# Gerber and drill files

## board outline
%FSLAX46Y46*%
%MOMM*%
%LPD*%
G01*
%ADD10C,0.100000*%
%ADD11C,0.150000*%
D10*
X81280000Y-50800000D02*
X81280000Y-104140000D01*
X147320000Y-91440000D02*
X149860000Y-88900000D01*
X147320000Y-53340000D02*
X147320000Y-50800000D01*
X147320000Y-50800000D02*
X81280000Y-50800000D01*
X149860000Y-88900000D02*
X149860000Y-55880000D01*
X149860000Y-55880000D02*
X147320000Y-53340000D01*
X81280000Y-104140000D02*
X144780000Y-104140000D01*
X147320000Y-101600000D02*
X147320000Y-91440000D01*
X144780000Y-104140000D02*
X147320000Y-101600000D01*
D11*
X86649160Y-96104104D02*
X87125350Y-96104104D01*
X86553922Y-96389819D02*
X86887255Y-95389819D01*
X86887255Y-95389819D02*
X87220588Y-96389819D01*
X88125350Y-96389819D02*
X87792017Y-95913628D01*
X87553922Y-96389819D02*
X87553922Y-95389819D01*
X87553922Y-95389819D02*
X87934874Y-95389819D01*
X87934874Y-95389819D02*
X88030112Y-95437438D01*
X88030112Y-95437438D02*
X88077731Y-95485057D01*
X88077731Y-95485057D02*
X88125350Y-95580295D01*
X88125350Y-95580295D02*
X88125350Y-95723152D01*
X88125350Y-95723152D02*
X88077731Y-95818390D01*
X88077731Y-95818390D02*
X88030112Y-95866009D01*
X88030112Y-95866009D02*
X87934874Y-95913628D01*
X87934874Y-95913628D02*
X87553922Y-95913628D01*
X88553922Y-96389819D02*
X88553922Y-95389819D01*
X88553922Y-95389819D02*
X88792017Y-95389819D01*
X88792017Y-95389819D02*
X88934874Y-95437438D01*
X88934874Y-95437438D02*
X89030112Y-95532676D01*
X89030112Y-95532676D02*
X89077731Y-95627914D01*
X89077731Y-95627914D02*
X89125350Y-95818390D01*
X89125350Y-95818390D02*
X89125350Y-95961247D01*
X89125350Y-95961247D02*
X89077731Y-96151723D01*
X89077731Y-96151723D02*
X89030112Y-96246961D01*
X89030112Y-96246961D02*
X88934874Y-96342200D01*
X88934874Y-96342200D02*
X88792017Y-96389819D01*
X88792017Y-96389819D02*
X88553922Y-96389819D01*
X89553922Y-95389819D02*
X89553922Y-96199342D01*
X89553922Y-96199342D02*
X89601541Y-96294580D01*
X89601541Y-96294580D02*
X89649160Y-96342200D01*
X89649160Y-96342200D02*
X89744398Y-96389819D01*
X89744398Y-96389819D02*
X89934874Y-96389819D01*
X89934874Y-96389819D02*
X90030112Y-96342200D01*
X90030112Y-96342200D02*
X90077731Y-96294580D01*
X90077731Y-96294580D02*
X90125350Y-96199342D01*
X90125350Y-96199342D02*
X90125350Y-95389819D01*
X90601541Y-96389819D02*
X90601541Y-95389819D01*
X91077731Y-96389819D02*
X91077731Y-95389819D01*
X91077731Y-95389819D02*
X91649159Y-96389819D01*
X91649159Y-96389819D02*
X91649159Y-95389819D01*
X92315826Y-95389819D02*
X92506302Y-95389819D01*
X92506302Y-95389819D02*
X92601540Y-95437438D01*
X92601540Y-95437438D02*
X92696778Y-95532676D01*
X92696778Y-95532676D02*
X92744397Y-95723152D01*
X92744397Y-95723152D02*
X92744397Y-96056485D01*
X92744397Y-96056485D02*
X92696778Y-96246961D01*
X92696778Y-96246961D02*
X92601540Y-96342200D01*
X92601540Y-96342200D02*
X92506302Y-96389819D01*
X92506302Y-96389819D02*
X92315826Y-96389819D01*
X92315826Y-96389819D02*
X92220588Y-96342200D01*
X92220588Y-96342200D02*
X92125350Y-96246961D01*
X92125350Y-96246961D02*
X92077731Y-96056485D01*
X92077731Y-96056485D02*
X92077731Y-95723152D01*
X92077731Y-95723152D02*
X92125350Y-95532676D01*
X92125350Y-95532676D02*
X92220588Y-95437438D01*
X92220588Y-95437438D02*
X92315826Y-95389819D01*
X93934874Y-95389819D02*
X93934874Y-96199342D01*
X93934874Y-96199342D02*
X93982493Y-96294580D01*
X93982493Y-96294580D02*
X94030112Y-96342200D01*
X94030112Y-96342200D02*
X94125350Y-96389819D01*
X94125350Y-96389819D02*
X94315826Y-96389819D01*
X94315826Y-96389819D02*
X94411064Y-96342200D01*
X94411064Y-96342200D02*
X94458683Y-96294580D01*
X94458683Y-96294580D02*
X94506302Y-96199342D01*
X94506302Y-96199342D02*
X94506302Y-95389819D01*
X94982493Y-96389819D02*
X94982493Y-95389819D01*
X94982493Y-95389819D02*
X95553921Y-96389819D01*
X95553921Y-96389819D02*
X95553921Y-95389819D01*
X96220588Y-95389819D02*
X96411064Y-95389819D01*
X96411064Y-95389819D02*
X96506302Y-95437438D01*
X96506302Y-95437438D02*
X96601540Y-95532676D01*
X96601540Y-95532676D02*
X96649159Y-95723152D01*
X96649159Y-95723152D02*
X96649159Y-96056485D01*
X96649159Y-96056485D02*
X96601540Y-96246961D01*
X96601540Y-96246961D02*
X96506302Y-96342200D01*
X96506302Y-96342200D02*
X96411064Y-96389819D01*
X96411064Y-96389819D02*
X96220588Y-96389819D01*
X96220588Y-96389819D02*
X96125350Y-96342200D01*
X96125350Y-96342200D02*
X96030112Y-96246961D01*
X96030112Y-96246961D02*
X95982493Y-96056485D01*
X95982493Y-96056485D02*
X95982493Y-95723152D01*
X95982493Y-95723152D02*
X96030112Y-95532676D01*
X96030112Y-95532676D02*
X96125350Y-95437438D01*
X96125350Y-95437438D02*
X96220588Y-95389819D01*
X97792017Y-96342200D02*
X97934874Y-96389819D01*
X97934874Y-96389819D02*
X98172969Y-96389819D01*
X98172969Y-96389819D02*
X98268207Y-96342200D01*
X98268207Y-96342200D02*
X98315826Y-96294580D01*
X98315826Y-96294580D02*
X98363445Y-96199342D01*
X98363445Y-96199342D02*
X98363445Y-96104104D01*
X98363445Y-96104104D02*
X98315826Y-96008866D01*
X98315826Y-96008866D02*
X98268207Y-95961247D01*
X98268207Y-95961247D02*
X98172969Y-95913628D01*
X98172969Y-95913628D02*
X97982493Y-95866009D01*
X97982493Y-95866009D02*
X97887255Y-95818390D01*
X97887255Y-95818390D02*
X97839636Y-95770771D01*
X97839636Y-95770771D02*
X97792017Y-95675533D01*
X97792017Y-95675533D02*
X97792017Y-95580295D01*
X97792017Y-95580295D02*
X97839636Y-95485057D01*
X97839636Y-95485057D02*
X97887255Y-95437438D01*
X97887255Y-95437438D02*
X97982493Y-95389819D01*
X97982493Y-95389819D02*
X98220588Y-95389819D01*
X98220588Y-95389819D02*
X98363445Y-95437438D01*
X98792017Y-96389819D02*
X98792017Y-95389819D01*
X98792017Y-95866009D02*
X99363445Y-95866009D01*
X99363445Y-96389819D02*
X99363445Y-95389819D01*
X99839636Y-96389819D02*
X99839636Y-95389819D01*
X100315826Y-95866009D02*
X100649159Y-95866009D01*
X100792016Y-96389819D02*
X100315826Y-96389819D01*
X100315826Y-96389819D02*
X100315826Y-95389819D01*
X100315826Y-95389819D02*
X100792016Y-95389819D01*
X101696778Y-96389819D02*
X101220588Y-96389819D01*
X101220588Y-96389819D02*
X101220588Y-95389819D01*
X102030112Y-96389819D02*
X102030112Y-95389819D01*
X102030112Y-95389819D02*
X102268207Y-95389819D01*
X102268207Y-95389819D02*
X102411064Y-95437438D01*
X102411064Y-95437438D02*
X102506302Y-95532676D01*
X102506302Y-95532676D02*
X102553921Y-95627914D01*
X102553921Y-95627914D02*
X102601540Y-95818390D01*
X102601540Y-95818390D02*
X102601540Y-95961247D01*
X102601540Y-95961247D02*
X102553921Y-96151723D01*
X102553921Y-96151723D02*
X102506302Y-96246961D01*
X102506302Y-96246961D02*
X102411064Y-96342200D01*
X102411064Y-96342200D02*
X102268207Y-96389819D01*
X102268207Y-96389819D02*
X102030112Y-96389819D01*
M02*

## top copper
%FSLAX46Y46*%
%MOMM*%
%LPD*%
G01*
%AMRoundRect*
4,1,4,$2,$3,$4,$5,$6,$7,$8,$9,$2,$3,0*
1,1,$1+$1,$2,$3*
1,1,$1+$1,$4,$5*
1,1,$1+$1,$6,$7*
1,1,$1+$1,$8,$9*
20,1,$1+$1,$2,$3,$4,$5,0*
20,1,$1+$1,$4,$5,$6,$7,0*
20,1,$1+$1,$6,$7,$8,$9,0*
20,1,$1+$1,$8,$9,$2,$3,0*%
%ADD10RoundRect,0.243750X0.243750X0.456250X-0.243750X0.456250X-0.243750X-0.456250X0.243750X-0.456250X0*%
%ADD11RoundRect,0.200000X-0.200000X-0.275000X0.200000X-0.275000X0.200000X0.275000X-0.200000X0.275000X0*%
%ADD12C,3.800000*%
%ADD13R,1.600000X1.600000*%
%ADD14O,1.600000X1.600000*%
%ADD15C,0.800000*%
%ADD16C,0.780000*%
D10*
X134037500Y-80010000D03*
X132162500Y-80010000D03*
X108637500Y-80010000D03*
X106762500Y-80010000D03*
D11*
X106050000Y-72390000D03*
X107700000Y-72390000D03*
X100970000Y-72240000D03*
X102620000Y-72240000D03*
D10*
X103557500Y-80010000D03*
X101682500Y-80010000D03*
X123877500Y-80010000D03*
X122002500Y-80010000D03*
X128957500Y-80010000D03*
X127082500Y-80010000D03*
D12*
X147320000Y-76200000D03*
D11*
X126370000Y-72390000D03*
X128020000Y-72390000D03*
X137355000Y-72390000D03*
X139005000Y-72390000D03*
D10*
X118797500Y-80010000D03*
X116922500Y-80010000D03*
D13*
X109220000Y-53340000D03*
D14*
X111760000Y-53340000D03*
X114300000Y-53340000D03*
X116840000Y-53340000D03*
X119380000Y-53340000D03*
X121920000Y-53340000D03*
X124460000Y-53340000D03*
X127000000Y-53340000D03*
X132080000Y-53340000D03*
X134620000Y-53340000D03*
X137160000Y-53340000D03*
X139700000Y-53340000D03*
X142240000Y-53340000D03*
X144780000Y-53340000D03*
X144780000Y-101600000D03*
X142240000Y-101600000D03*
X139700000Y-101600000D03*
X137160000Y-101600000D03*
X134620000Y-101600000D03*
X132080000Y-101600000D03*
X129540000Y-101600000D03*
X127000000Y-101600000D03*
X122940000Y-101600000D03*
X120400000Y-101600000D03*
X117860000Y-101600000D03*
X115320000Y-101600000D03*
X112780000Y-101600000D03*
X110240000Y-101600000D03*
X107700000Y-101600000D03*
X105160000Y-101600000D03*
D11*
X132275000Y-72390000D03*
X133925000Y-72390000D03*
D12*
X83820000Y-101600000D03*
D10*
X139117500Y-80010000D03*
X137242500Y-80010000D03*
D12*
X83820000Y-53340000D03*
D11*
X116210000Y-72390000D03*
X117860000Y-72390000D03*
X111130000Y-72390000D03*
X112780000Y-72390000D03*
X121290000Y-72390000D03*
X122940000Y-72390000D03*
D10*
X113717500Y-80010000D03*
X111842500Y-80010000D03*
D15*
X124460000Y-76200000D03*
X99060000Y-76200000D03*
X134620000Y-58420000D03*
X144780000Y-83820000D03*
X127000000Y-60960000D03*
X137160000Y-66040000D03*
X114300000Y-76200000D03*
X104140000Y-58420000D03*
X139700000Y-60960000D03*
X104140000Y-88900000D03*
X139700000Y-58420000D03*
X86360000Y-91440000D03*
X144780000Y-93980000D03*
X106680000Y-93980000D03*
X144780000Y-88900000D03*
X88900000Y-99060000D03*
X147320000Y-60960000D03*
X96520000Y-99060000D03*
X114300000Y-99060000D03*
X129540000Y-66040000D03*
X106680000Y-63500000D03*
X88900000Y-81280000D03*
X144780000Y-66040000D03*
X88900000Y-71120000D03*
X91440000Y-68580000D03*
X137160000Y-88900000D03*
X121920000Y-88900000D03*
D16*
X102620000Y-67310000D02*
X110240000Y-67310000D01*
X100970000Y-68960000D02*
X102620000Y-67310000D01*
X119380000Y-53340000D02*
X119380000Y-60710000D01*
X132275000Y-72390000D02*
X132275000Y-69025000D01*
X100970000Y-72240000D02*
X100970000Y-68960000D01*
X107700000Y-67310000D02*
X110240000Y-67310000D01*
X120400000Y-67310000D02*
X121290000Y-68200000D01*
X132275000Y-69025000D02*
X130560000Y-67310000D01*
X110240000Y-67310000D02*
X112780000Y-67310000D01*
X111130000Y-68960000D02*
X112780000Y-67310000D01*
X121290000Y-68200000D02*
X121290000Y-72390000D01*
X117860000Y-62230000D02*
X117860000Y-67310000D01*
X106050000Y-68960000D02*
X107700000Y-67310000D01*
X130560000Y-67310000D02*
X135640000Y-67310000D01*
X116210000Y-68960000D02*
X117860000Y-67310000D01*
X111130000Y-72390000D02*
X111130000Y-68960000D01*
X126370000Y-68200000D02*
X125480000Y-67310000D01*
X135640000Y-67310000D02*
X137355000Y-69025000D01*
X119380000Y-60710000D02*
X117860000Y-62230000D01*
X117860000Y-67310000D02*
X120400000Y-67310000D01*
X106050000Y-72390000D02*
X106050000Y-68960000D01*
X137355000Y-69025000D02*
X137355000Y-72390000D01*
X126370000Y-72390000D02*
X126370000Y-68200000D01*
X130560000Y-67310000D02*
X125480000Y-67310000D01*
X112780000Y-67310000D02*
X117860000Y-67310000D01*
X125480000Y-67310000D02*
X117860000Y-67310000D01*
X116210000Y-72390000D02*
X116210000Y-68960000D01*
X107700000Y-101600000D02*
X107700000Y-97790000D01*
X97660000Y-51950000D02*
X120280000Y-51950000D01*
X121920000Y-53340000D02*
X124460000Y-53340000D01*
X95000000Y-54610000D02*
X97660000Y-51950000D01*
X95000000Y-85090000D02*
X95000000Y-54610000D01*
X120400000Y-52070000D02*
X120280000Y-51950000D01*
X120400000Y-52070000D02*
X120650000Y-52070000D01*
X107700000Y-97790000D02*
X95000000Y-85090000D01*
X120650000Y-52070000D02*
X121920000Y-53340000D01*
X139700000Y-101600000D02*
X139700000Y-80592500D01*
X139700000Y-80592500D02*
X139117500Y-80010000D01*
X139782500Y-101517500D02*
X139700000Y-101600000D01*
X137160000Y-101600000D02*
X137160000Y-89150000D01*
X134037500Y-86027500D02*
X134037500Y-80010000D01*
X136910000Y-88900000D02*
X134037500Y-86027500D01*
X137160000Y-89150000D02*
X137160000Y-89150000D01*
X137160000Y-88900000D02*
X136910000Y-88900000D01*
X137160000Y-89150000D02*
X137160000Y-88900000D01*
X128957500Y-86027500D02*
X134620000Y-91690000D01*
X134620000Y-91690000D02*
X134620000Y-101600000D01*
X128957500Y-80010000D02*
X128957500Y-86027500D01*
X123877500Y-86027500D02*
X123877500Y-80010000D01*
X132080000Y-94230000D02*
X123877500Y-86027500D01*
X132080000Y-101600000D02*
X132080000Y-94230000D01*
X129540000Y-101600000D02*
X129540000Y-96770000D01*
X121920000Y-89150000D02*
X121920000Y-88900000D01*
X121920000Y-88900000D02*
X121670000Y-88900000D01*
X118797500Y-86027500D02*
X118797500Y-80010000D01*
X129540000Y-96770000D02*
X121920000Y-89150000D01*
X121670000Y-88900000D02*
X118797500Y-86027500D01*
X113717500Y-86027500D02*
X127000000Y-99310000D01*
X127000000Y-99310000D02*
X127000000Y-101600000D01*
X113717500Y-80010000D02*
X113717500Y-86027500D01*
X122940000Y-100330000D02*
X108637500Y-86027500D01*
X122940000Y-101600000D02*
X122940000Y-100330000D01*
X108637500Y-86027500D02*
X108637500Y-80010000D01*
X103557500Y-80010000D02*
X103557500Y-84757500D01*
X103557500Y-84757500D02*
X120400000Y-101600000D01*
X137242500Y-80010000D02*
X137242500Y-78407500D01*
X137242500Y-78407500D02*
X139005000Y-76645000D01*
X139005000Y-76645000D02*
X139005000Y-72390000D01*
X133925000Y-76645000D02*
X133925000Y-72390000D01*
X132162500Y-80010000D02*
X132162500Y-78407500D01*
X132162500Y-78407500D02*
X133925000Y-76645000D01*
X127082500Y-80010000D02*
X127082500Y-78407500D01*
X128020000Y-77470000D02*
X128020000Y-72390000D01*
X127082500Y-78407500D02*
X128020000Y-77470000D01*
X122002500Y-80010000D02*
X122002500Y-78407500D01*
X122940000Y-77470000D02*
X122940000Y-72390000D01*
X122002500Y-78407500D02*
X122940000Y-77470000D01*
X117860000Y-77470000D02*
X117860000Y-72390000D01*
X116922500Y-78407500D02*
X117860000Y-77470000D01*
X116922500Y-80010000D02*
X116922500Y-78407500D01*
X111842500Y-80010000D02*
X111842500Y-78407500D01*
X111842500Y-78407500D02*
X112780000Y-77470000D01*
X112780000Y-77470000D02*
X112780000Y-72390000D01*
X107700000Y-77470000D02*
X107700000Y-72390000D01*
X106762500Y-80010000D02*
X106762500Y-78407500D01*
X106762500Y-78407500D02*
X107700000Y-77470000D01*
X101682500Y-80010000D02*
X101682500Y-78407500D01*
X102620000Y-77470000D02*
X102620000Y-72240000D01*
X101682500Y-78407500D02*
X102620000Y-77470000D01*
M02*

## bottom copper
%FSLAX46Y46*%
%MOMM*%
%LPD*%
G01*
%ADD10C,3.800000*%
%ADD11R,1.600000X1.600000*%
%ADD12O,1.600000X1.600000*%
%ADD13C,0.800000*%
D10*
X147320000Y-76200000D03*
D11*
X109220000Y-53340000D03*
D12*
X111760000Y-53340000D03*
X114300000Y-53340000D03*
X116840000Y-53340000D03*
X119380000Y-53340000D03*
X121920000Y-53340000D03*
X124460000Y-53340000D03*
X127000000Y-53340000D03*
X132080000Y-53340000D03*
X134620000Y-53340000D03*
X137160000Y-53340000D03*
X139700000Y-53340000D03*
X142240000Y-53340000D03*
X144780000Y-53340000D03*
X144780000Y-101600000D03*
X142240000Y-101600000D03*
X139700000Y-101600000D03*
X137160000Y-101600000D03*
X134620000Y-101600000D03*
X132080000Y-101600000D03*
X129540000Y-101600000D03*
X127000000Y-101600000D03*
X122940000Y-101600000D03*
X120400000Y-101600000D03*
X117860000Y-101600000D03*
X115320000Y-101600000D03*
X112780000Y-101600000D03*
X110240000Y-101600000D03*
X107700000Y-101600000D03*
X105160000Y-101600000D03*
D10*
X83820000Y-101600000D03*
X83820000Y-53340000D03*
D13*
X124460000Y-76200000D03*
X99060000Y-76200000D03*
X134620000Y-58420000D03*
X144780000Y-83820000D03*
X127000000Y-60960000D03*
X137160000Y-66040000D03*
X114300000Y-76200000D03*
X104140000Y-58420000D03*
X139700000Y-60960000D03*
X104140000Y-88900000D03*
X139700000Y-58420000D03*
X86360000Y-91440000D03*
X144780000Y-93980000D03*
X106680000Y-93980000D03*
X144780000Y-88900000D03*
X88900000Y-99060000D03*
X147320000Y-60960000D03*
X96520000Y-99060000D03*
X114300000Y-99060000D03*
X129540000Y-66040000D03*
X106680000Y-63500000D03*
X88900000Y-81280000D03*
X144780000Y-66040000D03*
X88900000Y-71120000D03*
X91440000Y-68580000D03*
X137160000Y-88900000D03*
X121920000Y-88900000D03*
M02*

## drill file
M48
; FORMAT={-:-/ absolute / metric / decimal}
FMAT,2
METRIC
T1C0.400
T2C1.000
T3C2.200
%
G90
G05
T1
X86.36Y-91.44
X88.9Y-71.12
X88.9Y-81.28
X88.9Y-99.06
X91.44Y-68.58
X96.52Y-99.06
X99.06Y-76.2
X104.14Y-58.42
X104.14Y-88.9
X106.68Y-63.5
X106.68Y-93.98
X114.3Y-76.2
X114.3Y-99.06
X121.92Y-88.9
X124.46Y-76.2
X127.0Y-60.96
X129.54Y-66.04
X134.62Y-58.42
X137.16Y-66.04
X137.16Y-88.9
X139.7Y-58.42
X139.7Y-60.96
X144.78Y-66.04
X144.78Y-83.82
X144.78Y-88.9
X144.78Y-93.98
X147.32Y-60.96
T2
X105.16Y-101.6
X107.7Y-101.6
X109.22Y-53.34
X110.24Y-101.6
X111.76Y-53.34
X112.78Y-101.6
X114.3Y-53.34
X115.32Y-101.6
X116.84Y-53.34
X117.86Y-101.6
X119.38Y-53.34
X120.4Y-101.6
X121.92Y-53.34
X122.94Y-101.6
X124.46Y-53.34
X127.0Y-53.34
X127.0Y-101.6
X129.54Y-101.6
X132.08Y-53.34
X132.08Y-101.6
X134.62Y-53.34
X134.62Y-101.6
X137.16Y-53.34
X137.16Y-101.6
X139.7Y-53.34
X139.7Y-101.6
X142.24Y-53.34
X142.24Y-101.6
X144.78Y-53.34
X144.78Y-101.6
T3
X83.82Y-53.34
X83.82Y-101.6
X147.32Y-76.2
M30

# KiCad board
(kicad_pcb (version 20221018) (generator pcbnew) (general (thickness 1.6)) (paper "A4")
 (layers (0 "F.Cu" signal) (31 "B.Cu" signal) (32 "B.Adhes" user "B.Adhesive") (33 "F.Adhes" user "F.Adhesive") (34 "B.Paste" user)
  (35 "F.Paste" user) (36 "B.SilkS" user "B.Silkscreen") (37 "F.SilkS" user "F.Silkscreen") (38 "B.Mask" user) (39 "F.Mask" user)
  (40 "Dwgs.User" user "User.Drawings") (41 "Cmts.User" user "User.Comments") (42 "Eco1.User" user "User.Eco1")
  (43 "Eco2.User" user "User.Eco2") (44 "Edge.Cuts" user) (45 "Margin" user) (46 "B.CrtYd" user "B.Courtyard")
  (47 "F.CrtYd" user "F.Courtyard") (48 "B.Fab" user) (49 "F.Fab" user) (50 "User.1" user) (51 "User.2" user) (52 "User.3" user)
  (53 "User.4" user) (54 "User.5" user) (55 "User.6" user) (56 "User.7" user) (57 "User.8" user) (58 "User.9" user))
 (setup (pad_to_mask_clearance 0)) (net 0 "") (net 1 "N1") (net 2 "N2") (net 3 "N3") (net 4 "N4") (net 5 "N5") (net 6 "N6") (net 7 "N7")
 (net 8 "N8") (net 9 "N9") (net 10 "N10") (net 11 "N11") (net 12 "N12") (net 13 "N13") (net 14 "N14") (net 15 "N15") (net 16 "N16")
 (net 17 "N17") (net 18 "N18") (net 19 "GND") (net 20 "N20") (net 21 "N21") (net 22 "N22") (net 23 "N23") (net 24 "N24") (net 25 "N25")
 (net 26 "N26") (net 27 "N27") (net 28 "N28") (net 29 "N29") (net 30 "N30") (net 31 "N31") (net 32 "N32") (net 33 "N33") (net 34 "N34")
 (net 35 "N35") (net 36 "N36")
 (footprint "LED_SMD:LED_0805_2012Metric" (layer "F.Cu") (at 133.1 80.01 180)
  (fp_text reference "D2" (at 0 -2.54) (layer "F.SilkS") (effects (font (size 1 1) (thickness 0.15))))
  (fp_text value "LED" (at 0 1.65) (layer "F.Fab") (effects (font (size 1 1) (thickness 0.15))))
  (pad "1" smd roundrect (at -0.9375 0 180) (size 0.975 1.4) (layers "F.Cu" "F.Paste" "F.Mask") (roundrect_rratio 0.25) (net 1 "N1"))
  (pad "2" smd roundrect (at 0.9375 0 180) (size 0.975 1.4) (layers "F.Cu" "F.Paste" "F.Mask") (roundrect_rratio 0.25) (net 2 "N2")))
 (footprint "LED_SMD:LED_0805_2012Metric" (layer "F.Cu") (at 107.7 80.01 180)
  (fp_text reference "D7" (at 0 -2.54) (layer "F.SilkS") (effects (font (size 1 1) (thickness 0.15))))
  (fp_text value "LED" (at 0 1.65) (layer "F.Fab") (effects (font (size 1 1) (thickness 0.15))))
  (pad "1" smd roundrect (at -0.9375 0 180) (size 0.975 1.4) (layers "F.Cu" "F.Paste" "F.Mask") (roundrect_rratio 0.25) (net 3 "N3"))
  (pad "2" smd roundrect (at 0.9375 0 180) (size 0.975 1.4) (layers "F.Cu" "F.Paste" "F.Mask") (roundrect_rratio 0.25) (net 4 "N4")))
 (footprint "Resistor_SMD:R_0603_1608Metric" (layer "F.Cu") (at 106.875 72.39)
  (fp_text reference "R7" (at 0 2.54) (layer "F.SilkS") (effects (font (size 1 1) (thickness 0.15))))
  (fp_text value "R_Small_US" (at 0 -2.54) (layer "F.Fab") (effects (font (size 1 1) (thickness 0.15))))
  (pad "1" smd roundrect (at -0.825 0) (size 0.8 0.95) (layers "F.Cu" "F.Paste" "F.Mask") (roundrect_rratio 0.25) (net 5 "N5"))
  (pad "2" smd roundrect (at 0.825 0) (size 0.8 0.95) (layers "F.Cu" "F.Paste" "F.Mask") (roundrect_rratio 0.25) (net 4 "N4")))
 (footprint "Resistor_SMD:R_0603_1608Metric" (layer "F.Cu") (at 101.795 72.24)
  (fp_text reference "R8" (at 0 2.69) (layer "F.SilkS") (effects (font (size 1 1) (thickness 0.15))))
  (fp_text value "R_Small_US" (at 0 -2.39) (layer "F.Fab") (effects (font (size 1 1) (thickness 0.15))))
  (pad "1" smd roundrect (at -0.825 0) (size 0.8 0.95) (layers "F.Cu" "F.Paste" "F.Mask") (roundrect_rratio 0.25) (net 5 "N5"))
  (pad "2" smd roundrect (at 0.825 0) (size 0.8 0.95) (layers "F.Cu" "F.Paste" "F.Mask") (roundrect_rratio 0.25) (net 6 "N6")))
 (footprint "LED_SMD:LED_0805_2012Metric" (layer "F.Cu") (at 102.62 80.01 180)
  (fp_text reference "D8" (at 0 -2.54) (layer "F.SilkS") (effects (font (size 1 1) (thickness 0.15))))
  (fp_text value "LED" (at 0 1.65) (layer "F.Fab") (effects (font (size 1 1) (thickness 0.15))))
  (pad "1" smd roundrect (at -0.9375 0 180) (size 0.975 1.4) (layers "F.Cu" "F.Paste" "F.Mask") (roundrect_rratio 0.25) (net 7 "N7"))
  (pad "2" smd roundrect (at 0.9375 0 180) (size 0.975 1.4) (layers "F.Cu" "F.Paste" "F.Mask") (roundrect_rratio 0.25) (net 6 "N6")))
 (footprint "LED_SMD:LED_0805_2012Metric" (layer "F.Cu") (at 122.94 80.01 180)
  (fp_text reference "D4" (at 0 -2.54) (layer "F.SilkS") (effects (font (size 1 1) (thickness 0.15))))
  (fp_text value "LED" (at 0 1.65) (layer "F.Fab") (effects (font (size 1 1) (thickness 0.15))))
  (pad "1" smd roundrect (at -0.9375 0 180) (size 0.975 1.4) (layers "F.Cu" "F.Paste" "F.Mask") (roundrect_rratio 0.25) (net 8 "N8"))
  (pad "2" smd roundrect (at 0.9375 0 180) (size 0.975 1.4) (layers "F.Cu" "F.Paste" "F.Mask") (roundrect_rratio 0.25) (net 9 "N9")))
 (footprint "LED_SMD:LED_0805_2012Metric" (layer "F.Cu") (at 128.02 80.01 180)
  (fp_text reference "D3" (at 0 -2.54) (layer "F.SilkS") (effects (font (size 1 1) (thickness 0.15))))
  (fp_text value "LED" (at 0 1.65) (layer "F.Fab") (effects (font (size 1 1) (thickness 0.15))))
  (pad "1" smd roundrect (at -0.9375 0 180) (size 0.975 1.4) (layers "F.Cu" "F.Paste" "F.Mask") (roundrect_rratio 0.25) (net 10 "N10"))
  (pad "2" smd roundrect (at 0.9375 0 180) (size 0.975 1.4) (layers "F.Cu" "F.Paste" "F.Mask") (roundrect_rratio 0.25) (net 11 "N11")))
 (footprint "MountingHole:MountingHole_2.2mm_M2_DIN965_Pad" (layer "F.Cu") (at 147.32 76.2)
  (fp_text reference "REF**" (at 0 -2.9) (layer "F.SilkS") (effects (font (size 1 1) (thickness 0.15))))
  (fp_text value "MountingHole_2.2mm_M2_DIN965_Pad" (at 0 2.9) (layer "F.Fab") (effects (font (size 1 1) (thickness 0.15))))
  (pad "1" thru_hole circle (at 0 0) (size 3.8 3.8) (drill 2.2) (layers "*.Cu" "*.Mask")))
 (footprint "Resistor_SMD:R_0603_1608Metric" (layer "F.Cu") (at 127.195 72.39)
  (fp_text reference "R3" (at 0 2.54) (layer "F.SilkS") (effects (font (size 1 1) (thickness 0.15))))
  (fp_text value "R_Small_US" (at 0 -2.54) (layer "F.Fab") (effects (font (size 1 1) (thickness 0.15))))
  (pad "1" smd roundrect (at -0.825 0) (size 0.8 0.95) (layers "F.Cu" "F.Paste" "F.Mask") (roundrect_rratio 0.25) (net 5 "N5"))
  (pad "2" smd roundrect (at 0.825 0) (size 0.8 0.95) (layers "F.Cu" "F.Paste" "F.Mask") (roundrect_rratio 0.25) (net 11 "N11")))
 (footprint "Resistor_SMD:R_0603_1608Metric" (layer "F.Cu") (at 138.18 72.39)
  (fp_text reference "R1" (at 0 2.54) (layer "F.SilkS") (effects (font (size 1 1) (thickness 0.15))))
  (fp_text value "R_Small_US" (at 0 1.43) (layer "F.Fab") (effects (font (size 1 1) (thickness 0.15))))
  (pad "1" smd roundrect (at -0.825 0) (size 0.8 0.95) (layers "F.Cu" "F.Paste" "F.Mask") (roundrect_rratio 0.25) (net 5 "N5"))
  (pad "2" smd roundrect (at 0.825 0) (size 0.8 0.95) (layers "F.Cu" "F.Paste" "F.Mask") (roundrect_rratio 0.25) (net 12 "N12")))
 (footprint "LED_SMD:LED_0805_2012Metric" (layer "F.Cu") (at 117.86 80.01 180)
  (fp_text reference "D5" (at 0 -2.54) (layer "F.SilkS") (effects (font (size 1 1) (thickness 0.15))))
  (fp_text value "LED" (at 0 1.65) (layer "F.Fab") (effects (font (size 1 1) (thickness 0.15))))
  (pad "1" smd roundrect (at -0.9375 0 180) (size 0.975 1.4) (layers "F.Cu" "F.Paste" "F.Mask") (roundrect_rratio 0.25) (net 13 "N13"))
  (pad "2" smd roundrect (at 0.9375 0 180) (size 0.975 1.4) (layers "F.Cu" "F.Paste" "F.Mask") (roundrect_rratio 0.25) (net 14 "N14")))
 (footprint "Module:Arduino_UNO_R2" (layer "F.Cu") (at 109.22 53.34)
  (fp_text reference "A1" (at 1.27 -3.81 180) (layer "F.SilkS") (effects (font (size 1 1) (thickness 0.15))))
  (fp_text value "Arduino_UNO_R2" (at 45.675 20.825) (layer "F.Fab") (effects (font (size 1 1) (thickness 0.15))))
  (pad "1" thru_hole rect (at 0 0 90) (size 1.6 1.6) (drill 1) (layers "*.Cu" "*.Mask") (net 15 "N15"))
  (pad "2" thru_hole oval (at 2.54 0 90) (size 1.6 1.6) (drill 1) (layers "*.Cu" "*.Mask") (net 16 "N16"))
  (pad "3" thru_hole oval (at 5.08 0 90) (size 1.6 1.6) (drill 1) (layers "*.Cu" "*.Mask") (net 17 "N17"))
  (pad "4" thru_hole oval (at 7.62 0 90) (size 1.6 1.6) (drill 1) (layers "*.Cu" "*.Mask") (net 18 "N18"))
  (pad "5" thru_hole oval (at 10.16 0 90) (size 1.6 1.6) (drill 1) (layers "*.Cu" "*.Mask") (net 5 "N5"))
  (pad "6" thru_hole oval (at 12.7 0 90) (size 1.6 1.6) (drill 1) (layers "*.Cu" "*.Mask") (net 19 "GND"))
  (pad "7" thru_hole oval (at 15.24 0 90) (size 1.6 1.6) (drill 1) (layers "*.Cu" "*.Mask") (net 19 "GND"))
  (pad "8" thru_hole oval (at 17.78 0 90) (size 1.6 1.6) (drill 1) (layers "*.Cu" "*.Mask") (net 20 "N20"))
  (pad "9" thru_hole oval (at 22.86 0 90) (size 1.6 1.6) (drill 1) (layers "*.Cu" "*.Mask") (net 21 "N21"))
  (pad "10" thru_hole oval (at 25.4 0 90) (size 1.6 1.6) (drill 1) (layers "*.Cu" "*.Mask") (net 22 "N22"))
  (pad "11" thru_hole oval (at 27.94 0 90) (size 1.6 1.6) (drill 1) (layers "*.Cu" "*.Mask") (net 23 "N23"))
  (pad "12" thru_hole oval (at 30.48 0 90) (size 1.6 1.6) (drill 1) (layers "*.Cu" "*.Mask") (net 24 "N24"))
  (pad "13" thru_hole oval (at 33.02 0 90) (size 1.6 1.6) (drill 1) (layers "*.Cu" "*.Mask") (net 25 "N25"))
  (pad "14" thru_hole oval (at 35.56 0 90) (size 1.6 1.6) (drill 1) (layers "*.Cu" "*.Mask") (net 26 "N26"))
  (pad "15" thru_hole oval (at 35.56 48.26 90) (size 1.6 1.6) (drill 1) (layers "*.Cu" "*.Mask") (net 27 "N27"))
  (pad "16" thru_hole oval (at 33.02 48.26 90) (size 1.6 1.6) (drill 1) (layers "*.Cu" "*.Mask") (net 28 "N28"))
  (pad "17" thru_hole oval (at 30.48 48.26 90) (size 1.6 1.6) (drill 1) (layers "*.Cu" "*.Mask") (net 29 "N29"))
  (pad "18" thru_hole oval (at 27.94 48.26 90) (size 1.6 1.6) (drill 1) (layers "*.Cu" "*.Mask") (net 1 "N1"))
  (pad "19" thru_hole oval (at 25.4 48.26 90) (size 1.6 1.6) (drill 1) (layers "*.Cu" "*.Mask") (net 10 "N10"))
  (pad "20" thru_hole oval (at 22.86 48.26 90) (size 1.6 1.6) (drill 1) (layers "*.Cu" "*.Mask") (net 8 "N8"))
  (pad "21" thru_hole oval (at 20.32 48.26 90) (size 1.6 1.6) (drill 1) (layers "*.Cu" "*.Mask") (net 13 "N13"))
  (pad "22" thru_hole oval (at 17.78 48.26 90) (size 1.6 1.6) (drill 1) (layers "*.Cu" "*.Mask") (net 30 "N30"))
  (pad "23" thru_hole oval (at 13.72 48.26 90) (size 1.6 1.6) (drill 1) (layers "*.Cu" "*.Mask") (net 3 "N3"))
  (pad "24" thru_hole oval (at 11.18 48.26 90) (size 1.6 1.6) (drill 1) (layers "*.Cu" "*.Mask") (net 7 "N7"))
  (pad "25" thru_hole oval (at 8.64 48.26 90) (size 1.6 1.6) (drill 1) (layers "*.Cu" "*.Mask") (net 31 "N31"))
  (pad "26" thru_hole oval (at 6.1 48.26 90) (size 1.6 1.6) (drill 1) (layers "*.Cu" "*.Mask") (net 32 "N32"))
  (pad "27" thru_hole oval (at 3.56 48.26 90) (size 1.6 1.6) (drill 1) (layers "*.Cu" "*.Mask") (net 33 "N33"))
  (pad "28" thru_hole oval (at 1.02 48.26 90) (size 1.6 1.6) (drill 1) (layers "*.Cu" "*.Mask") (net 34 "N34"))
  (pad "29" thru_hole oval (at -1.52 48.26 90) (size 1.6 1.6) (drill 1) (layers "*.Cu" "*.Mask") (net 19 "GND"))
  (pad "30" thru_hole oval (at -4.06 48.26 90) (size 1.6 1.6) (drill 1) (layers "*.Cu" "*.Mask") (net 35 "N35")))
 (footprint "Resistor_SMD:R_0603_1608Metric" (layer "F.Cu") (at 133.1 72.39)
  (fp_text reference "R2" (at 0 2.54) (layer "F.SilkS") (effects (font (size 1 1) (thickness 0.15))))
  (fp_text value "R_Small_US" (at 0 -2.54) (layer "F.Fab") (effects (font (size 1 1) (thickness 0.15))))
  (pad "1" smd roundrect (at -0.825 0) (size 0.8 0.95) (layers "F.Cu" "F.Paste" "F.Mask") (roundrect_rratio 0.25) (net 5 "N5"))
  (pad "2" smd roundrect (at 0.825 0) (size 0.8 0.95) (layers "F.Cu" "F.Paste" "F.Mask") (roundrect_rratio 0.25) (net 2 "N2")))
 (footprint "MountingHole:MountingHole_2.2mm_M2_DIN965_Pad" (layer "F.Cu") (at 83.82 101.6)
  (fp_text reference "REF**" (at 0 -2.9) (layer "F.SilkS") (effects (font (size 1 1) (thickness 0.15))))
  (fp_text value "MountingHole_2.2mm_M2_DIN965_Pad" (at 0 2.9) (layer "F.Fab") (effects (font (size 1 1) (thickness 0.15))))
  (pad "1" thru_hole circle (at 0 0) (size 3.8 3.8) (drill 2.2) (layers "*.Cu" "*.Mask")))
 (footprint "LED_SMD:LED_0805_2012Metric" (layer "F.Cu") (at 138.18 80.01 180)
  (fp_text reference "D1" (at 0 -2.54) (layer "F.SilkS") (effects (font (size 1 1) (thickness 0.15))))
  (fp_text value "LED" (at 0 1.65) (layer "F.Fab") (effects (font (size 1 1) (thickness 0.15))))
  (pad "1" smd roundrect (at -0.9375 0 180) (size 0.975 1.4) (layers "F.Cu" "F.Paste" "F.Mask") (roundrect_rratio 0.25) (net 29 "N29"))
  (pad "2" smd roundrect (at 0.9375 0 180) (size 0.975 1.4) (layers "F.Cu" "F.Paste" "F.Mask") (roundrect_rratio 0.25) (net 12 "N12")))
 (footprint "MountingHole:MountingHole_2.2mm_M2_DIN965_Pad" (layer "F.Cu") (at 83.82 53.34)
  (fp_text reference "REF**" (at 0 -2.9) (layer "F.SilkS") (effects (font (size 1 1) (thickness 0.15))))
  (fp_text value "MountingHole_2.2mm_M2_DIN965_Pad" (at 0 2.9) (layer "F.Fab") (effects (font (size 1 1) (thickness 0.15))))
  (pad "1" thru_hole circle (at 0 0) (size 3.8 3.8) (drill 2.2) (layers "*.Cu" "*.Mask")))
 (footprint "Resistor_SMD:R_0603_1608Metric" (layer "F.Cu") (at 117.035 72.39)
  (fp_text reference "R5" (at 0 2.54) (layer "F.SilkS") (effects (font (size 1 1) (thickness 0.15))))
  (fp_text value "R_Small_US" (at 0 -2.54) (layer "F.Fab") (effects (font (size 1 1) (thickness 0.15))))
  (pad "1" smd roundrect (at -0.825 0) (size 0.8 0.95) (layers "F.Cu" "F.Paste" "F.Mask") (roundrect_rratio 0.25) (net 5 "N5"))
  (pad "2" smd roundrect (at 0.825 0) (size 0.8 0.95) (layers "F.Cu" "F.Paste" "F.Mask") (roundrect_rratio 0.25) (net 14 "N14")))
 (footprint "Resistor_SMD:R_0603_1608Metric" (layer "F.Cu") (at 111.955 72.39)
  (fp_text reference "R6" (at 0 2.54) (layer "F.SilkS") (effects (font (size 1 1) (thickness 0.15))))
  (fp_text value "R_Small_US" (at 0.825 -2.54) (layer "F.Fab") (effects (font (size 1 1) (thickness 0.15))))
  (pad "1" smd roundrect (at -0.825 0) (size 0.8 0.95) (layers "F.Cu" "F.Paste" "F.Mask") (roundrect_rratio 0.25) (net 5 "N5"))
  (pad "2" smd roundrect (at 0.825 0) (size 0.8 0.95) (layers "F.Cu" "F.Paste" "F.Mask") (roundrect_rratio 0.25) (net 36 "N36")))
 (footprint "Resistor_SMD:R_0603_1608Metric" (layer "F.Cu") (at 122.115 72.39)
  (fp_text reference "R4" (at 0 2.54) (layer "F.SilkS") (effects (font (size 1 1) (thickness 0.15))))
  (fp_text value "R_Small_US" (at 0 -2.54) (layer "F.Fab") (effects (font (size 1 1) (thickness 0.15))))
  (pad "1" smd roundrect (at -0.825 0) (size 0.8 0.95) (layers "F.Cu" "F.Paste" "F.Mask") (roundrect_rratio 0.25) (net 5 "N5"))
  (pad "2" smd roundrect (at 0.825 0) (size 0.8 0.95) (layers "F.Cu" "F.Paste" "F.Mask") (roundrect_rratio 0.25) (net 9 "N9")))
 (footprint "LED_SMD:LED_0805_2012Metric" (layer "F.Cu") (at 112.78 80.01 180)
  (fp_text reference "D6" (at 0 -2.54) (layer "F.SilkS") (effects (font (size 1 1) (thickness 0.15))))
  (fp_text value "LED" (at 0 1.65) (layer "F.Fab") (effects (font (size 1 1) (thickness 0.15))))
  (pad "1" smd roundrect (at -0.9375 0 180) (size 0.975 1.4) (layers "F.Cu" "F.Paste" "F.Mask") (roundrect_rratio 0.25) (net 30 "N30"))
  (pad "2" smd roundrect (at 0.9375 0 180) (size 0.975 1.4) (layers "F.Cu" "F.Paste" "F.Mask") (roundrect_rratio 0.25) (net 36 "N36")))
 (gr_line (start 81.28 50.8) (end 81.28 104.14) (stroke (width 0.1) (type default)) (layer "Edge.Cuts"))
 (gr_line (start 147.32 91.44) (end 149.86 88.9) (stroke (width 0.1) (type default)) (layer "Edge.Cuts"))
 (gr_line (start 147.32 53.34) (end 147.32 50.8) (stroke (width 0.1) (type default)) (layer "Edge.Cuts"))
 (gr_line (start 147.32 50.8) (end 81.28 50.8) (stroke (width 0.1) (type default)) (layer "Edge.Cuts"))
 (gr_line (start 149.86 88.9) (end 149.86 55.88) (stroke (width 0.1) (type default)) (layer "Edge.Cuts"))
 (gr_line (start 149.86 55.88) (end 147.32 53.34) (stroke (width 0.1) (type default)) (layer "Edge.Cuts"))
 (gr_line (start 81.28 104.14) (end 144.78 104.14) (stroke (width 0.1) (type default)) (layer "Edge.Cuts"))
 (gr_line (start 147.32 101.6) (end 147.32 91.44) (stroke (width 0.1) (type default)) (layer "Edge.Cuts"))
 (gr_line (start 144.78 104.14) (end 147.32 101.6) (stroke (width 0.1) (type default)) (layer "Edge.Cuts"))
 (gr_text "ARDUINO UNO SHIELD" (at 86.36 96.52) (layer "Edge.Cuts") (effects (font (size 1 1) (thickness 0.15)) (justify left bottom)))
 (via (at 124.46 76.2) (size 0.8) (drill 0.4) (layers "F.Cu" "B.Cu") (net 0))
 (via (at 99.06 76.2) (size 0.8) (drill 0.4) (layers "F.Cu" "B.Cu") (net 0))
 (via (at 134.62 58.42) (size 0.8) (drill 0.4) (layers "F.Cu" "B.Cu") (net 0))
 (via (at 144.78 83.82) (size 0.8) (drill 0.4) (layers "F.Cu" "B.Cu") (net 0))
 (via (at 127 60.96) (size 0.8) (drill 0.4) (layers "F.Cu" "B.Cu") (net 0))
 (via (at 137.16 66.04) (size 0.8) (drill 0.4) (layers "F.Cu" "B.Cu") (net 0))
 (via (at 114.3 76.2) (size 0.8) (drill 0.4) (layers "F.Cu" "B.Cu") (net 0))
 (via (at 104.14 58.42) (size 0.8) (drill 0.4) (layers "F.Cu" "B.Cu") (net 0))
 (via (at 139.7 60.96) (size 0.8) (drill 0.4) (layers "F.Cu" "B.Cu") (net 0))
 (via (at 104.14 88.9) (size 0.8) (drill 0.4) (layers "F.Cu" "B.Cu") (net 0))
 (via (at 139.7 58.42) (size 0.8) (drill 0.4) (layers "F.Cu" "B.Cu") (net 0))
 (via (at 86.36 91.44) (size 0.8) (drill 0.4) (layers "F.Cu" "B.Cu") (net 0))
 (via (at 144.78 93.98) (size 0.8) (drill 0.4) (layers "F.Cu" "B.Cu") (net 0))
 (via (at 106.68 93.98) (size 0.8) (drill 0.4) (layers "F.Cu" "B.Cu") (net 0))
 (via (at 144.78 88.9) (size 0.8) (drill 0.4) (layers "F.Cu" "B.Cu") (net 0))
 (via (at 88.9 99.06) (size 0.8) (drill 0.4) (layers "F.Cu" "B.Cu") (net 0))
 (via (at 147.32 60.96) (size 0.8) (drill 0.4) (layers "F.Cu" "B.Cu") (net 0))
 (via (at 96.52 99.06) (size 0.8) (drill 0.4) (layers "F.Cu" "B.Cu") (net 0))
 (via (at 114.3 99.06) (size 0.8) (drill 0.4) (layers "F.Cu" "B.Cu") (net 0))
 (via (at 129.54 66.04) (size 0.8) (drill 0.4) (layers "F.Cu" "B.Cu") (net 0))
 (via (at 106.68 63.5) (size 0.8) (drill 0.4) (layers "F.Cu" "B.Cu") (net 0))
 (via (at 88.9 81.28) (size 0.8) (drill 0.4) (layers "F.Cu" "B.Cu") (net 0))
 (via (at 144.78 66.04) (size 0.8) (drill 0.4) (layers "F.Cu" "B.Cu") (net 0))
 (via (at 88.9 71.12) (size 0.8) (drill 0.4) (layers "F.Cu" "B.Cu") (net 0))
 (via (at 91.44 68.58) (size 0.8) (drill 0.4) (layers "F.Cu" "B.Cu") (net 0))
 (segment (start 102.62 67.31) (end 110.24 67.31) (width 0.78) (layer "F.Cu") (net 5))
 (segment (start 100.97 68.96) (end 102.62 67.31) (width 0.78) (layer "F.Cu") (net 5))
 (segment (start 119.38 53.34) (end 119.38 60.71) (width 0.78) (layer "F.Cu") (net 5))
 (segment (start 132.275 72.39) (end 132.275 69.025) (width 0.78) (layer "F.Cu") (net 5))
 (segment (start 100.97 72.24) (end 100.97 68.96) (width 0.78) (layer "F.Cu") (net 5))
 (segment (start 107.7 67.31) (end 110.24 67.31) (width 0.78) (layer "F.Cu") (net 5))
 (segment (start 120.4 67.31) (end 121.29 68.2) (width 0.78) (layer "F.Cu") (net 5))
 (segment (start 132.275 69.025) (end 130.56 67.31) (width 0.78) (layer "F.Cu") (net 5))
 (segment (start 110.24 67.31) (end 112.78 67.31) (width 0.78) (layer "F.Cu") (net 5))
 (segment (start 111.13 68.96) (end 112.78 67.31) (width 0.78) (layer "F.Cu") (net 5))
 (segment (start 121.29 68.2) (end 121.29 72.39) (width 0.78) (layer "F.Cu") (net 5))
 (segment (start 117.86 62.23) (end 117.86 67.31) (width 0.78) (layer "F.Cu") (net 5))
 (segment (start 106.05 68.96) (end 107.7 67.31) (width 0.78) (layer "F.Cu") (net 5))
 (segment (start 130.56 67.31) (end 135.64 67.31) (width 0.78) (layer "F.Cu") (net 5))
 (segment (start 116.21 68.96) (end 117.86 67.31) (width 0.78) (layer "F.Cu") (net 5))
 (segment (start 111.13 72.39) (end 111.13 68.96) (width 0.78) (layer "F.Cu") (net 5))
 (segment (start 126.37 68.2) (end 125.48 67.31) (width 0.78) (layer "F.Cu") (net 5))
 (segment (start 135.64 67.31) (end 137.355 69.025) (width 0.78) (layer "F.Cu") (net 5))
 (segment (start 119.38 60.71) (end 117.86 62.23) (width 0.78) (layer "F.Cu") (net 5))
 (segment (start 117.86 67.31) (end 120.4 67.31) (width 0.78) (layer "F.Cu") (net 5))
 (segment (start 106.05 72.39) (end 106.05 68.96) (width 0.78) (layer "F.Cu") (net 5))
 (segment (start 137.355 69.025) (end 137.355 72.39) (width 0.78) (layer "F.Cu") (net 5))
 (segment (start 126.37 72.39) (end 126.37 68.2) (width 0.78) (layer "F.Cu") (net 5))
 (segment (start 130.56 67.31) (end 125.48 67.31) (width 0.78) (layer "F.Cu") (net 5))
 (segment (start 112.78 67.31) (end 117.86 67.31) (width 0.78) (layer "F.Cu") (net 5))
 (segment (start 125.48 67.31) (end 117.86 67.31) (width 0.78) (layer "F.Cu") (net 5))
 (segment (start 116.21 72.39) (end 116.21 68.96) (width 0.78) (layer "F.Cu") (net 5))
 (segment (start 107.7 101.6) (end 107.7 97.79) (width 0.78) (layer "F.Cu") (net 19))
 (segment (start 97.66 51.95) (end 120.28 51.95) (width 0.78) (layer "F.Cu") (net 19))
 (segment (start 121.92 53.34) (end 124.46 53.34) (width 0.78) (layer "F.Cu") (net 19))
 (segment (start 95 54.61) (end 97.66 51.95) (width 0.78) (layer "F.Cu") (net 19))
 (segment (start 95 85.09) (end 95 54.61) (width 0.78) (layer "F.Cu") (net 19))
 (segment (start 120.4 52.07) (end 120.28 51.95) (width 0.78) (layer "F.Cu") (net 19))
 (segment (start 120.4 52.07) (end 120.65 52.07) (width 0.78) (layer "F.Cu") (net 19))
 (segment (start 107.7 97.79) (end 95 85.09) (width 0.78) (layer "F.Cu") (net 19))
 (segment (start 120.65 52.07) (end 121.92 53.34) (width 0.78) (layer "F.Cu") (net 19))
 (segment (start 139.7 101.6) (end 139.7 80.5925) (width 0.78) (layer "F.Cu") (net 29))
 (segment (start 139.7 80.5925) (end 139.1175 80.01) (width 0.78) (layer "F.Cu") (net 29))
 (segment (start 139.7825 101.5175) (end 139.7 101.6) (width 0.78) (layer "F.Cu") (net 29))
 (segment (start 137.16 101.6) (end 137.16 89.15) (width 0.78) (layer "F.Cu") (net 1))
 (segment (start 134.0375 86.0275) (end 134.0375 80.01) (width 0.78) (layer "F.Cu") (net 1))
 (segment (start 136.91 88.9) (end 134.0375 86.0275) (width 0.78) (layer "F.Cu") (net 1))
 (segment (start 137.16 89.15) (end 137.16 89.15) (width 0.78) (layer "F.Cu") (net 1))
 (segment (start 137.16 88.9) (end 136.91 88.9) (width 0.78) (layer "F.Cu") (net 1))
 (segment (start 137.16 89.15) (end 137.16 88.9) (width 0.78) (layer "F.Cu") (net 1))
 (via (at 137.16 88.9) (size 0.8) (drill 0.4) (layers "F.Cu" "B.Cu") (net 1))
 (segment (start 128.9575 86.0275) (end 134.62 91.69) (width 0.78) (layer "F.Cu") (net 10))
 (segment (start 134.62 91.69) (end 134.62 101.6) (width 0.78) (layer "F.Cu") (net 10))
 (segment (start 128.9575 80.01) (end 128.9575 86.0275) (width 0.78) (layer "F.Cu") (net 10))
 (segment (start 123.8775 86.0275) (end 123.8775 80.01) (width 0.78) (layer "F.Cu") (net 8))
 (segment (start 132.08 94.23) (end 123.8775 86.0275) (width 0.78) (layer "F.Cu") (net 8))
 (segment (start 132.08 101.6) (end 132.08 94.23) (width 0.78) (layer "F.Cu") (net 8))
 (segment (start 129.54 101.6) (end 129.54 96.77) (width 0.78) (layer "F.Cu") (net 13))
 (segment (start 121.92 89.15) (end 121.92 88.9) (width 0.78) (layer "F.Cu") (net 13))
 (segment (start 121.92 88.9) (end 121.67 88.9) (width 0.78) (layer "F.Cu") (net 13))
 (segment (start 118.7975 86.0275) (end 118.7975 80.01) (width 0.78) (layer "F.Cu") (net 13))
 (segment (start 129.54 96.77) (end 121.92 89.15) (width 0.78) (layer "F.Cu") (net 13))
 (segment (start 121.67 88.9) (end 118.7975 86.0275) (width 0.78) (layer "F.Cu") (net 13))
 (via (at 121.92 88.9) (size 0.8) (drill 0.4) (layers "F.Cu" "B.Cu") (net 13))
 (segment (start 113.7175 86.0275) (end 127 99.31) (width 0.78) (layer "F.Cu") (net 30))
 (segment (start 127 99.31) (end 127 101.6) (width 0.78) (layer "F.Cu") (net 30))
 (segment (start 113.7175 80.01) (end 113.7175 86.0275) (width 0.78) (layer "F.Cu") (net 30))
 (segment (start 122.94 100.33) (end 108.6375 86.0275) (width 0.78) (layer "F.Cu") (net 3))
 (segment (start 122.94 101.6) (end 122.94 100.33) (width 0.78) (layer "F.Cu") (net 3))
 (segment (start 108.6375 86.0275) (end 108.6375 80.01) (width 0.78) (layer "F.Cu") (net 3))
 (segment (start 103.5575 80.01) (end 103.5575 84.7575) (width 0.78) (layer "F.Cu") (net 7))
 (segment (start 103.5575 84.7575) (end 120.4 101.6) (width 0.78) (layer "F.Cu") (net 7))
 (segment (start 137.2425 80.01) (end 137.2425 78.4075) (width 0.78) (layer "F.Cu") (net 12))
 (segment (start 137.2425 78.4075) (end 139.005 76.645) (width 0.78) (layer "F.Cu") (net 12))
 (segment (start 139.005 76.645) (end 139.005 72.39) (width 0.78) (layer "F.Cu") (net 12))
 (segment (start 133.925 76.645) (end 133.925 72.39) (width 0.78) (layer "F.Cu") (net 2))
 (segment (start 132.1625 80.01) (end 132.1625 78.4075) (width 0.78) (layer "F.Cu") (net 2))
 (segment (start 132.1625 78.4075) (end 133.925 76.645) (width 0.78) (layer "F.Cu") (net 2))
 (segment (start 127.0825 80.01) (end 127.0825 78.4075) (width 0.78) (layer "F.Cu") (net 11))
 (segment (start 128.02 77.47) (end 128.02 72.39) (width 0.78) (layer "F.Cu") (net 11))
 (segment (start 127.0825 78.4075) (end 128.02 77.47) (width 0.78) (layer "F.Cu") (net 11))
 (segment (start 122.0025 80.01) (end 122.0025 78.4075) (width 0.78) (layer "F.Cu") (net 9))
 (segment (start 122.94 77.47) (end 122.94 72.39) (width 0.78) (layer "F.Cu") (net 9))
 (segment (start 122.0025 78.4075) (end 122.94 77.47) (width 0.78) (layer "F.Cu") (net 9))
 (segment (start 117.86 77.47) (end 117.86 72.39) (width 0.78) (layer "F.Cu") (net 14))
 (segment (start 116.9225 78.4075) (end 117.86 77.47) (width 0.78) (layer "F.Cu") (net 14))
 (segment (start 116.9225 80.01) (end 116.9225 78.4075) (width 0.78) (layer "F.Cu") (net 14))
 (segment (start 111.8425 80.01) (end 111.8425 78.4075) (width 0.78) (layer "F.Cu") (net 36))
 (segment (start 111.8425 78.4075) (end 112.78 77.47) (width 0.78) (layer "F.Cu") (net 36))
 (segment (start 112.78 77.47) (end 112.78 72.39) (width 0.78) (layer "F.Cu") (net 36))
 (segment (start 107.7 77.47) (end 107.7 72.39) (width 0.78) (layer "F.Cu") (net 4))
 (segment (start 106.7625 80.01) (end 106.7625 78.4075) (width 0.78) (layer "F.Cu") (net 4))
 (segment (start 106.7625 78.4075) (end 107.7 77.47) (width 0.78) (layer "F.Cu") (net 4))
 (segment (start 101.6825 80.01) (end 101.6825 78.4075) (width 0.78) (layer "F.Cu") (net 6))
 (segment (start 102.62 77.47) (end 102.62 72.24) (width 0.78) (layer "F.Cu") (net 6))
 (segment (start 101.6825 78.4075) (end 102.62 77.47) (width 0.78) (layer "F.Cu") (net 6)))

